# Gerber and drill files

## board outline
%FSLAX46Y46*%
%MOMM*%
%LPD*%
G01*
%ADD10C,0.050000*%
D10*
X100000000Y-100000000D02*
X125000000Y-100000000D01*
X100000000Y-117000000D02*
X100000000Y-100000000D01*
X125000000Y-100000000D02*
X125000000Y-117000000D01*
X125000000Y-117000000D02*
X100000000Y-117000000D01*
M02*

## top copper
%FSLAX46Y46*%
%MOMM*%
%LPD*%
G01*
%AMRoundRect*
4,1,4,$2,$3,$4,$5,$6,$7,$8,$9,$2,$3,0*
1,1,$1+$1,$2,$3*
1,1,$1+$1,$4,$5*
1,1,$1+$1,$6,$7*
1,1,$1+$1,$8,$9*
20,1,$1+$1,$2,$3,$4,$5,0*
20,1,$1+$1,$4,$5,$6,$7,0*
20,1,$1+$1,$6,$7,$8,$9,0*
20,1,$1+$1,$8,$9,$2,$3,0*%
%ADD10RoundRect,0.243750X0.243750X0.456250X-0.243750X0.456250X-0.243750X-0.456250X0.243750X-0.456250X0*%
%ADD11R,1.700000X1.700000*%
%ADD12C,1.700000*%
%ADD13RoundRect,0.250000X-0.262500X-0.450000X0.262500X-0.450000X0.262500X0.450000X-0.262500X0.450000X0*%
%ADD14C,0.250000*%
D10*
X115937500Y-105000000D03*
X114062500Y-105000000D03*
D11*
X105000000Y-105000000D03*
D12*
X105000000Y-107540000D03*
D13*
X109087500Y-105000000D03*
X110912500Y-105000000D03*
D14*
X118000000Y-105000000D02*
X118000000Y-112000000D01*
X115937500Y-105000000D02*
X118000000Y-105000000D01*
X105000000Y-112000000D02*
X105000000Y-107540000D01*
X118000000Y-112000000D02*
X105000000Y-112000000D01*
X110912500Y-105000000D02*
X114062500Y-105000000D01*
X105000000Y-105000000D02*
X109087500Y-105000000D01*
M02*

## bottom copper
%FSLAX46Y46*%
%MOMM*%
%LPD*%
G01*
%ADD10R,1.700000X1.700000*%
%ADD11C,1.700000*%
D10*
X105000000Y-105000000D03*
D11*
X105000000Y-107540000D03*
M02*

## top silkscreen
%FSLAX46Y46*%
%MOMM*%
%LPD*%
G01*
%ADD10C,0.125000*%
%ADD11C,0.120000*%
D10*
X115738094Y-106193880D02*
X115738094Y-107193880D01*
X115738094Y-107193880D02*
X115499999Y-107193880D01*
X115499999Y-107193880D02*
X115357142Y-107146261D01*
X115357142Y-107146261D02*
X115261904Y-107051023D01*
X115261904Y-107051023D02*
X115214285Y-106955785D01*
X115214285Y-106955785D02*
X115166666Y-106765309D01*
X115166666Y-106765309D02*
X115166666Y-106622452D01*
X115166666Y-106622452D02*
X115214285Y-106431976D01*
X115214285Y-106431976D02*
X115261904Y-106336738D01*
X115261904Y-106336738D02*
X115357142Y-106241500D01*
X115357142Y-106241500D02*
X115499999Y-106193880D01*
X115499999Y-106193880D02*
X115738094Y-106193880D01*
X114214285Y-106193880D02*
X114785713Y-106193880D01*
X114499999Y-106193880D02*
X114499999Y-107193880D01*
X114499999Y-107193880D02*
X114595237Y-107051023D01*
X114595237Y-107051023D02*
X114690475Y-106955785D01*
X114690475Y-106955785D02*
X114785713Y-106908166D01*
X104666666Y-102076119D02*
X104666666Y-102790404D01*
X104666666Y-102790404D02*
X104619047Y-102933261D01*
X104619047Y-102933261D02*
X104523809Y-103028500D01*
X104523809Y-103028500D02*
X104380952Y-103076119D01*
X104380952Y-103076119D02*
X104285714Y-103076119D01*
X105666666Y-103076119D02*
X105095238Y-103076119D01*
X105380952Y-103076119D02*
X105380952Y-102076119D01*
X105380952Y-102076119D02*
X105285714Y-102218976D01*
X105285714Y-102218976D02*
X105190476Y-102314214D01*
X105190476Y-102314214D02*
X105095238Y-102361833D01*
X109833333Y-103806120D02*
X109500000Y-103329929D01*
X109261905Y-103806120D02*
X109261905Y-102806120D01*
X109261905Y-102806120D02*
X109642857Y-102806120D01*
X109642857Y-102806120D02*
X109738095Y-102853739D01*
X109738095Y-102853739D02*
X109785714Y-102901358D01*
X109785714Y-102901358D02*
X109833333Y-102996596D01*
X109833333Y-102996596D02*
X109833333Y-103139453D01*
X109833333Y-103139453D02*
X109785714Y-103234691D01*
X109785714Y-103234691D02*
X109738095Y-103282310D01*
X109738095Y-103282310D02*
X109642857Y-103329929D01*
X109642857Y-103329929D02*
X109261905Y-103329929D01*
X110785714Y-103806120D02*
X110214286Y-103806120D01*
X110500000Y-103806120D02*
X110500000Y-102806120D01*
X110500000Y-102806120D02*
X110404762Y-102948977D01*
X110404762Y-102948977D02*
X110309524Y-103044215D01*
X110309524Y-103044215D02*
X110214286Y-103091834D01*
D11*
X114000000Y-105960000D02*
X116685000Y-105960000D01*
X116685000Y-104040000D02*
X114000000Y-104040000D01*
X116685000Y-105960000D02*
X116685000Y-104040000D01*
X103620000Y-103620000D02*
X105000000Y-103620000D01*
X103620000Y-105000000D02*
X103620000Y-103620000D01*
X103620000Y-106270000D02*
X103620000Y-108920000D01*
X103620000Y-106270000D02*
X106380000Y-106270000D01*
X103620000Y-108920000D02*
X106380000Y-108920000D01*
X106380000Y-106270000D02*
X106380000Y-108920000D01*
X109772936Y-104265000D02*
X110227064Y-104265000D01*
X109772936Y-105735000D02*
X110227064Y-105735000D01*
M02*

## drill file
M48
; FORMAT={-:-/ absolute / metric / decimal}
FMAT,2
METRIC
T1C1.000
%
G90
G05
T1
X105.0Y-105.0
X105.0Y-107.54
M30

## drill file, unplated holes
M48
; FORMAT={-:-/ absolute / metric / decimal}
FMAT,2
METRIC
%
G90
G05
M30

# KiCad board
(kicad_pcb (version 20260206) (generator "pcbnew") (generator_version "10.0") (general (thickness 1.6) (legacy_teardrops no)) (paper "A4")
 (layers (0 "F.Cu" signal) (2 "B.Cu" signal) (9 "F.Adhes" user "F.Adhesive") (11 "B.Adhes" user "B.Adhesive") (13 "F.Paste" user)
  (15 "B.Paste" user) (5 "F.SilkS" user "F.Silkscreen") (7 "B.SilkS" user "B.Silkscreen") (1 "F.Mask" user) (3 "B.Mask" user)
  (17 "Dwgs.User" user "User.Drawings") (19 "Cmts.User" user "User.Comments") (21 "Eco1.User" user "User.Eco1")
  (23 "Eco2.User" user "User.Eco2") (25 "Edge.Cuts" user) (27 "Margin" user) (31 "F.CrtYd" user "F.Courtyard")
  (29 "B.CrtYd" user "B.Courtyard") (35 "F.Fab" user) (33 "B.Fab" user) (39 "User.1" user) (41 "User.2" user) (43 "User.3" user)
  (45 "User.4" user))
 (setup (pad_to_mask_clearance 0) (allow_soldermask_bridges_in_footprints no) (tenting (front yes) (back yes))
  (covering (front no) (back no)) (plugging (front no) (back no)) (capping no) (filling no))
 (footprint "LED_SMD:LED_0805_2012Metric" (layer "F.Cu") (at 115 105 180)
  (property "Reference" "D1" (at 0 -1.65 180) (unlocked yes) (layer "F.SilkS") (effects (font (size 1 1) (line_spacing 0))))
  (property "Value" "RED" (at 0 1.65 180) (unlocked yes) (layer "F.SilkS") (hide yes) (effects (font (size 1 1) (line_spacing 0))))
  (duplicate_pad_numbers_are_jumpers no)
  (fp_line (start 1 -0.96) (end -1.685 -0.96) (stroke (width 0.12) (type default)) (layer "F.SilkS"))
  (fp_line (start -1.685 0.96) (end 1 0.96) (stroke (width 0.12) (type default)) (layer "F.SilkS"))
  (fp_line (start -1.685 -0.96) (end -1.685 0.96) (stroke (width 0.12) (type default)) (layer "F.SilkS"))
  (pad "1" smd roundrect (at -0.9375 0 180) (size 0.975 1.4) (layers "F.Cu" "F.Mask" "F.Paste") (roundrect_rratio 0.25) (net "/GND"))
  (pad "2" smd roundrect (at 0.9375 0 180) (size 0.975 1.4) (layers "F.Cu" "F.Mask" "F.Paste") (roundrect_rratio 0.25) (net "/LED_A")))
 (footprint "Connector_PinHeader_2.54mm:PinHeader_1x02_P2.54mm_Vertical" (layer "F.Cu") (at 105 105)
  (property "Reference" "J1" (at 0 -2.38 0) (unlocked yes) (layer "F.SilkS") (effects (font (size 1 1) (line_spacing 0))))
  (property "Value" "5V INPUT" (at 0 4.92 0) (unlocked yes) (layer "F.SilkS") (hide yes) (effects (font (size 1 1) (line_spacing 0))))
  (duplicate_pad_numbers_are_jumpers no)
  (fp_line (start -1.38 -1.38) (end 0 -1.38) (stroke (width 0.12) (type default)) (layer "F.SilkS"))
  (fp_line (start -1.38 0) (end -1.38 -1.38) (stroke (width 0.12) (type default)) (layer "F.SilkS"))
  (fp_line (start -1.38 1.27) (end -1.38 3.92) (stroke (width 0.12) (type default)) (layer "F.SilkS"))
  (fp_line (start -1.38 1.27) (end 1.38 1.27) (stroke (width 0.12) (type default)) (layer "F.SilkS"))
  (fp_line (start -1.38 3.92) (end 1.38 3.92) (stroke (width 0.12) (type default)) (layer "F.SilkS"))
  (fp_line (start 1.38 1.27) (end 1.38 3.92) (stroke (width 0.12) (type default)) (layer "F.SilkS"))
  (pad "1" thru_hole rect (at 0 0) (size 1.7 1.7) (drill 1) (layers "*.Cu" "*.Mask") (remove_unused_layers no) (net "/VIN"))
  (pad "2" thru_hole circle (at 0 2.54) (size 1.7 1.7) (drill 1) (layers "*.Cu" "*.Mask") (remove_unused_layers no) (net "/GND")))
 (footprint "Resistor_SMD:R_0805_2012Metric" (layer "F.Cu") (at 110 105)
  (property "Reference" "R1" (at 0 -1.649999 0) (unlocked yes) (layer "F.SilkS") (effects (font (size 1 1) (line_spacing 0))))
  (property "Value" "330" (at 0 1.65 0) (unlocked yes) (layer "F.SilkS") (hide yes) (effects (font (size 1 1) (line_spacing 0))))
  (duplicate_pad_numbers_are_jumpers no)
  (fp_line (start -0.227064 -0.735) (end 0.227064 -0.735) (stroke (width 0.12) (type default)) (layer "F.SilkS"))
  (fp_line (start -0.227064 0.735) (end 0.227064 0.735) (stroke (width 0.12) (type default)) (layer "F.SilkS"))
  (pad "1" smd roundrect (at -0.9125 0) (size 1.025 1.4) (layers "F.Cu" "F.Mask" "F.Paste") (roundrect_rratio 0.243902) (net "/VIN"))
  (pad "2" smd roundrect (at 0.9125 0) (size 1.025 1.4) (layers "F.Cu" "F.Mask" "F.Paste") (roundrect_rratio 0.243902) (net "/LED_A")))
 (gr_line (start 100 100) (end 125 100) (stroke (width 0.05) (type default)) (layer "Edge.Cuts"))
 (gr_line (start 100 117) (end 100 100) (stroke (width 0.05) (type default)) (layer "Edge.Cuts"))
 (gr_line (start 125 100) (end 125 117) (stroke (width 0.05) (type default)) (layer "Edge.Cuts"))
 (gr_line (start 125 117) (end 100 117) (stroke (width 0.05) (type default)) (layer "Edge.Cuts"))
 (segment (start 118 105) (end 118 112) (width 0.25) (layer "F.Cu") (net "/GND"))
 (segment (start 115.9375 105) (end 118 105) (width 0.25) (layer "F.Cu") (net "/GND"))
 (segment (start 105 112) (end 105 107.54) (width 0.25) (layer "F.Cu") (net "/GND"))
 (segment (start 118 112) (end 105 112) (width 0.25) (layer "F.Cu") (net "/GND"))
 (segment (start 110.9125 105) (end 114.0625 105) (width 0.25) (layer "F.Cu") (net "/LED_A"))
 (segment (start 105 105) (end 109.0875 105) (width 0.25) (layer "F.Cu") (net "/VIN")))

